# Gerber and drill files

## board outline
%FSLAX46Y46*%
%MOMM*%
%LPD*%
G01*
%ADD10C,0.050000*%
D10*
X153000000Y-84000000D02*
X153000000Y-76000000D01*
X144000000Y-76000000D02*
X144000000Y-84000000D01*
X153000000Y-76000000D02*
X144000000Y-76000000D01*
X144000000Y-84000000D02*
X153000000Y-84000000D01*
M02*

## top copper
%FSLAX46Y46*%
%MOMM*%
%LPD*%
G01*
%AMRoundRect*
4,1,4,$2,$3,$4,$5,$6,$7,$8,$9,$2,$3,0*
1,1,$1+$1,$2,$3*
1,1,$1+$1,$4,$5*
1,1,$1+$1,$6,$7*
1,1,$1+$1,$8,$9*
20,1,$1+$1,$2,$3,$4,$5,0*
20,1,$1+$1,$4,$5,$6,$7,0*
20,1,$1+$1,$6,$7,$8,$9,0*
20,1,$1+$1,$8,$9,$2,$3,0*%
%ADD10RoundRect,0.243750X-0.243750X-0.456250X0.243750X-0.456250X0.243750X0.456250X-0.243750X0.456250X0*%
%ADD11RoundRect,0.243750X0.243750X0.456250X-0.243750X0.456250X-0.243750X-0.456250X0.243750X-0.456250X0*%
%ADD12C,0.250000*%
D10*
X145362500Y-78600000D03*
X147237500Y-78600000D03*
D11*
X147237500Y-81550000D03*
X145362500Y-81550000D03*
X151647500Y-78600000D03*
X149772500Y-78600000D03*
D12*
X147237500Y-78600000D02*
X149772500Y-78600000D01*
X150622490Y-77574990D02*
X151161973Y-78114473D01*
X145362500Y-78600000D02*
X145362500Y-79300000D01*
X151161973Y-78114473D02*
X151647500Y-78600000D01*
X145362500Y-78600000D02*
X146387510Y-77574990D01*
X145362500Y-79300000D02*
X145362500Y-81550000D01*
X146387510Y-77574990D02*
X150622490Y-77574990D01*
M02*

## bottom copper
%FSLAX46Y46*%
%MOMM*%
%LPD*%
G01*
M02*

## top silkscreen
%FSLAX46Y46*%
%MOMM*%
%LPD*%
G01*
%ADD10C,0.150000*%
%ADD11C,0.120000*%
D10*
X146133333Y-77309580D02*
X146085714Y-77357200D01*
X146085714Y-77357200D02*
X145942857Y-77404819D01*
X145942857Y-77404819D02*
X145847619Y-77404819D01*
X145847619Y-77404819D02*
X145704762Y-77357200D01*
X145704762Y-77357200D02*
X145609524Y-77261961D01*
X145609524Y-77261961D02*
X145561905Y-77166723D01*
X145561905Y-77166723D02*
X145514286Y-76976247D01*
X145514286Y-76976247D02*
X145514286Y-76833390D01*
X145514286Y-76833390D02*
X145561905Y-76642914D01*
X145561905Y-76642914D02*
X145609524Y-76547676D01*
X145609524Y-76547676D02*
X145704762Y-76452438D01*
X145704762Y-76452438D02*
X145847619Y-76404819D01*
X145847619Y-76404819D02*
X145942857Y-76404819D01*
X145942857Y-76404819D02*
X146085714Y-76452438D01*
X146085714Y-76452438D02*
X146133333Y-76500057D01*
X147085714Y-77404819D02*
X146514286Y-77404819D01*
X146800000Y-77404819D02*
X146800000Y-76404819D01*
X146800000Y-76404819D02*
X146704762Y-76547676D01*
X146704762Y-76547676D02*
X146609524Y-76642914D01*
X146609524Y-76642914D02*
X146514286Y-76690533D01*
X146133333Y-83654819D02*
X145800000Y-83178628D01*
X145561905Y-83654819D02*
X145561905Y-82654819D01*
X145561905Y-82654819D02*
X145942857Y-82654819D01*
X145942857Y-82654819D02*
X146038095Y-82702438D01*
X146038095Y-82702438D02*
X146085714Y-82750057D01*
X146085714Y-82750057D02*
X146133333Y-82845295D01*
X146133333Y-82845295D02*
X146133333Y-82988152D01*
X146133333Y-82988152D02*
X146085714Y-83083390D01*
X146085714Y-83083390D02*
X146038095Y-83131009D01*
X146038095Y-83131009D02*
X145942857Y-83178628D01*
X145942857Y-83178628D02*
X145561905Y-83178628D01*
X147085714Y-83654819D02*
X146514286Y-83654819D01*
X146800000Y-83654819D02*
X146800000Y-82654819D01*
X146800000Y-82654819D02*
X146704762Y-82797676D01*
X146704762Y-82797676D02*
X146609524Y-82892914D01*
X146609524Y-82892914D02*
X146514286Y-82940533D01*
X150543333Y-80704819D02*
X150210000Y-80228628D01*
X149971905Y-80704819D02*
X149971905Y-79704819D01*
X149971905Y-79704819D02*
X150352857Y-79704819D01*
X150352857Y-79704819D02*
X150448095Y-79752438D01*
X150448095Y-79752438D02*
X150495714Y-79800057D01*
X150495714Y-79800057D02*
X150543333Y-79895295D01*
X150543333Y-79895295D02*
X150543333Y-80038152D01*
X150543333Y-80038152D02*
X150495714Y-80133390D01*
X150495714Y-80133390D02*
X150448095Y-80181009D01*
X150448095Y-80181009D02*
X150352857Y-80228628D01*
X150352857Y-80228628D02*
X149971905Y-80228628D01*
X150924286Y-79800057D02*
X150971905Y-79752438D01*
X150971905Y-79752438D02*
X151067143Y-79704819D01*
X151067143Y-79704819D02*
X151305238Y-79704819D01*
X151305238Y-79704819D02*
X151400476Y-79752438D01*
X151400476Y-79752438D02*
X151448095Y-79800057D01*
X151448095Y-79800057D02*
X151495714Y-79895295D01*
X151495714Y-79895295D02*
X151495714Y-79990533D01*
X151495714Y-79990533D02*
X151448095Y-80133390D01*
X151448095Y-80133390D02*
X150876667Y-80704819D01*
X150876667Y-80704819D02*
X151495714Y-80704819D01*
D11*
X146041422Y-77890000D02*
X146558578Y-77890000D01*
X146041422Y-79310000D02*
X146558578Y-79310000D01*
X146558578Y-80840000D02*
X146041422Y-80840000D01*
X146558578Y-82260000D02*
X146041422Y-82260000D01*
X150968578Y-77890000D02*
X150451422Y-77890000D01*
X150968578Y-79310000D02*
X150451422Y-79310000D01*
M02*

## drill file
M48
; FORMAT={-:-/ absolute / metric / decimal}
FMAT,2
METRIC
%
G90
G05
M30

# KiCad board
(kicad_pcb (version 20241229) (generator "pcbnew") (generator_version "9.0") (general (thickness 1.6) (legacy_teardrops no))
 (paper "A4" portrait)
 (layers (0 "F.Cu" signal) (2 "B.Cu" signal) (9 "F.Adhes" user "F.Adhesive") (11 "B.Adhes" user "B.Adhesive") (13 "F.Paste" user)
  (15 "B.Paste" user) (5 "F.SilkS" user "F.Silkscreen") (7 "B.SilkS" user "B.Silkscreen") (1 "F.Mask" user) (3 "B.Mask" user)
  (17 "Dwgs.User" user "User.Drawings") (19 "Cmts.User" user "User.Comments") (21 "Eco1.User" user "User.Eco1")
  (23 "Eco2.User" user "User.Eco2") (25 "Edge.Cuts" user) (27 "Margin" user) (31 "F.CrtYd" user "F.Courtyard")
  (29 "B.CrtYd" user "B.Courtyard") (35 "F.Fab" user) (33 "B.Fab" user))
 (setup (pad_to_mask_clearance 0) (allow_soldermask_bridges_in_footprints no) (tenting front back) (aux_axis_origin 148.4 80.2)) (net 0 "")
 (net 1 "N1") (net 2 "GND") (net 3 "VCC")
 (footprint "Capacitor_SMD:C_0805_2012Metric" (layer "F.Cu") (at 146.3 78.6)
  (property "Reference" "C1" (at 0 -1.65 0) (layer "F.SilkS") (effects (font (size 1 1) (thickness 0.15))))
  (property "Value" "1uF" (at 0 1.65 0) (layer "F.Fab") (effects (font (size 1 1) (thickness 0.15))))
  (fp_line (start -0.258578 -0.71) (end 0.258578 -0.71) (stroke (width 0.12) (type solid)) (layer "F.SilkS"))
  (fp_line (start -0.258578 0.71) (end 0.258578 0.71) (stroke (width 0.12) (type solid)) (layer "F.SilkS"))
  (pad "1" smd roundrect (at -0.9375 0) (size 0.975 1.4) (layers "F.Cu" "F.Mask" "F.Paste") (roundrect_rratio 0.25) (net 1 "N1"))
  (pad "2" smd roundrect (at 0.9375 0) (size 0.975 1.4) (layers "F.Cu" "F.Mask" "F.Paste") (roundrect_rratio 0.25) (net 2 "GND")))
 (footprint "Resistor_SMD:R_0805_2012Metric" (layer "F.Cu") (at 146.3 81.55 180)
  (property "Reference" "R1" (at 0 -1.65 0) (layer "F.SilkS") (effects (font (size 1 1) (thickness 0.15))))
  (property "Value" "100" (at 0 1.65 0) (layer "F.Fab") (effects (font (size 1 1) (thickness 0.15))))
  (fp_line (start -0.258578 0.71) (end 0.258578 0.71) (stroke (width 0.12) (type solid)) (layer "F.SilkS"))
  (fp_line (start -0.258578 -0.71) (end 0.258578 -0.71) (stroke (width 0.12) (type solid)) (layer "F.SilkS"))
  (pad "1" smd roundrect (at -0.9375 0 180) (size 0.975 1.4) (layers "F.Cu" "F.Mask" "F.Paste") (roundrect_rratio 0.25) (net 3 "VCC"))
  (pad "2" smd roundrect (at 0.9375 0 180) (size 0.975 1.4) (layers "F.Cu" "F.Mask" "F.Paste") (roundrect_rratio 0.25) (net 1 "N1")))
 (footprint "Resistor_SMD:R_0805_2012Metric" (layer "F.Cu") (at 150.71 78.6 180)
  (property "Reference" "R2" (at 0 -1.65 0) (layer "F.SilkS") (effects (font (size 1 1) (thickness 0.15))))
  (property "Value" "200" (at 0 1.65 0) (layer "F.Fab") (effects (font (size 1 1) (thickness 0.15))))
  (fp_line (start -0.258578 0.71) (end 0.258578 0.71) (stroke (width 0.12) (type solid)) (layer "F.SilkS"))
  (fp_line (start -0.258578 -0.71) (end 0.258578 -0.71) (stroke (width 0.12) (type solid)) (layer "F.SilkS"))
  (pad "1" smd roundrect (at -0.9375 0 180) (size 0.975 1.4) (layers "F.Cu" "F.Mask" "F.Paste") (roundrect_rratio 0.25) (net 1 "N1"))
  (pad "2" smd roundrect (at 0.9375 0 180) (size 0.975 1.4) (layers "F.Cu" "F.Mask" "F.Paste") (roundrect_rratio 0.25) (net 2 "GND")))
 (gr_line (start 153 84) (end 153 76) (stroke (width 0.05) (type solid)) (layer "Edge.Cuts"))
 (gr_line (start 144 76) (end 144 84) (stroke (width 0.05) (type solid)) (layer "Edge.Cuts"))
 (gr_line (start 153 76) (end 144 76) (stroke (width 0.05) (type solid)) (layer "Edge.Cuts"))
 (gr_line (start 144 84) (end 153 84) (stroke (width 0.05) (type solid)) (layer "Edge.Cuts"))
 (segment (start 147.2375 78.6) (end 149.7725 78.6) (width 0.25) (layer "F.Cu") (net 2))
 (segment (start 150.62249 77.57499) (end 151.161973 78.114473) (width 0.25) (layer "F.Cu") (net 1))
 (segment (start 145.3625 78.6) (end 145.3625 79.3) (width 0.25) (layer "F.Cu") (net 1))
 (segment (start 151.161973 78.114473) (end 151.6475 78.6) (width 0.25) (layer "F.Cu") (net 1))
 (segment (start 145.3625 78.6) (end 146.38751 77.57499) (width 0.25) (layer "F.Cu") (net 1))
 (segment (start 145.3625 79.3) (end 145.3625 81.55) (width 0.25) (layer "F.Cu") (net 1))
 (segment (start 146.38751 77.57499) (end 150.62249 77.57499) (width 0.25) (layer "F.Cu") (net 1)))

